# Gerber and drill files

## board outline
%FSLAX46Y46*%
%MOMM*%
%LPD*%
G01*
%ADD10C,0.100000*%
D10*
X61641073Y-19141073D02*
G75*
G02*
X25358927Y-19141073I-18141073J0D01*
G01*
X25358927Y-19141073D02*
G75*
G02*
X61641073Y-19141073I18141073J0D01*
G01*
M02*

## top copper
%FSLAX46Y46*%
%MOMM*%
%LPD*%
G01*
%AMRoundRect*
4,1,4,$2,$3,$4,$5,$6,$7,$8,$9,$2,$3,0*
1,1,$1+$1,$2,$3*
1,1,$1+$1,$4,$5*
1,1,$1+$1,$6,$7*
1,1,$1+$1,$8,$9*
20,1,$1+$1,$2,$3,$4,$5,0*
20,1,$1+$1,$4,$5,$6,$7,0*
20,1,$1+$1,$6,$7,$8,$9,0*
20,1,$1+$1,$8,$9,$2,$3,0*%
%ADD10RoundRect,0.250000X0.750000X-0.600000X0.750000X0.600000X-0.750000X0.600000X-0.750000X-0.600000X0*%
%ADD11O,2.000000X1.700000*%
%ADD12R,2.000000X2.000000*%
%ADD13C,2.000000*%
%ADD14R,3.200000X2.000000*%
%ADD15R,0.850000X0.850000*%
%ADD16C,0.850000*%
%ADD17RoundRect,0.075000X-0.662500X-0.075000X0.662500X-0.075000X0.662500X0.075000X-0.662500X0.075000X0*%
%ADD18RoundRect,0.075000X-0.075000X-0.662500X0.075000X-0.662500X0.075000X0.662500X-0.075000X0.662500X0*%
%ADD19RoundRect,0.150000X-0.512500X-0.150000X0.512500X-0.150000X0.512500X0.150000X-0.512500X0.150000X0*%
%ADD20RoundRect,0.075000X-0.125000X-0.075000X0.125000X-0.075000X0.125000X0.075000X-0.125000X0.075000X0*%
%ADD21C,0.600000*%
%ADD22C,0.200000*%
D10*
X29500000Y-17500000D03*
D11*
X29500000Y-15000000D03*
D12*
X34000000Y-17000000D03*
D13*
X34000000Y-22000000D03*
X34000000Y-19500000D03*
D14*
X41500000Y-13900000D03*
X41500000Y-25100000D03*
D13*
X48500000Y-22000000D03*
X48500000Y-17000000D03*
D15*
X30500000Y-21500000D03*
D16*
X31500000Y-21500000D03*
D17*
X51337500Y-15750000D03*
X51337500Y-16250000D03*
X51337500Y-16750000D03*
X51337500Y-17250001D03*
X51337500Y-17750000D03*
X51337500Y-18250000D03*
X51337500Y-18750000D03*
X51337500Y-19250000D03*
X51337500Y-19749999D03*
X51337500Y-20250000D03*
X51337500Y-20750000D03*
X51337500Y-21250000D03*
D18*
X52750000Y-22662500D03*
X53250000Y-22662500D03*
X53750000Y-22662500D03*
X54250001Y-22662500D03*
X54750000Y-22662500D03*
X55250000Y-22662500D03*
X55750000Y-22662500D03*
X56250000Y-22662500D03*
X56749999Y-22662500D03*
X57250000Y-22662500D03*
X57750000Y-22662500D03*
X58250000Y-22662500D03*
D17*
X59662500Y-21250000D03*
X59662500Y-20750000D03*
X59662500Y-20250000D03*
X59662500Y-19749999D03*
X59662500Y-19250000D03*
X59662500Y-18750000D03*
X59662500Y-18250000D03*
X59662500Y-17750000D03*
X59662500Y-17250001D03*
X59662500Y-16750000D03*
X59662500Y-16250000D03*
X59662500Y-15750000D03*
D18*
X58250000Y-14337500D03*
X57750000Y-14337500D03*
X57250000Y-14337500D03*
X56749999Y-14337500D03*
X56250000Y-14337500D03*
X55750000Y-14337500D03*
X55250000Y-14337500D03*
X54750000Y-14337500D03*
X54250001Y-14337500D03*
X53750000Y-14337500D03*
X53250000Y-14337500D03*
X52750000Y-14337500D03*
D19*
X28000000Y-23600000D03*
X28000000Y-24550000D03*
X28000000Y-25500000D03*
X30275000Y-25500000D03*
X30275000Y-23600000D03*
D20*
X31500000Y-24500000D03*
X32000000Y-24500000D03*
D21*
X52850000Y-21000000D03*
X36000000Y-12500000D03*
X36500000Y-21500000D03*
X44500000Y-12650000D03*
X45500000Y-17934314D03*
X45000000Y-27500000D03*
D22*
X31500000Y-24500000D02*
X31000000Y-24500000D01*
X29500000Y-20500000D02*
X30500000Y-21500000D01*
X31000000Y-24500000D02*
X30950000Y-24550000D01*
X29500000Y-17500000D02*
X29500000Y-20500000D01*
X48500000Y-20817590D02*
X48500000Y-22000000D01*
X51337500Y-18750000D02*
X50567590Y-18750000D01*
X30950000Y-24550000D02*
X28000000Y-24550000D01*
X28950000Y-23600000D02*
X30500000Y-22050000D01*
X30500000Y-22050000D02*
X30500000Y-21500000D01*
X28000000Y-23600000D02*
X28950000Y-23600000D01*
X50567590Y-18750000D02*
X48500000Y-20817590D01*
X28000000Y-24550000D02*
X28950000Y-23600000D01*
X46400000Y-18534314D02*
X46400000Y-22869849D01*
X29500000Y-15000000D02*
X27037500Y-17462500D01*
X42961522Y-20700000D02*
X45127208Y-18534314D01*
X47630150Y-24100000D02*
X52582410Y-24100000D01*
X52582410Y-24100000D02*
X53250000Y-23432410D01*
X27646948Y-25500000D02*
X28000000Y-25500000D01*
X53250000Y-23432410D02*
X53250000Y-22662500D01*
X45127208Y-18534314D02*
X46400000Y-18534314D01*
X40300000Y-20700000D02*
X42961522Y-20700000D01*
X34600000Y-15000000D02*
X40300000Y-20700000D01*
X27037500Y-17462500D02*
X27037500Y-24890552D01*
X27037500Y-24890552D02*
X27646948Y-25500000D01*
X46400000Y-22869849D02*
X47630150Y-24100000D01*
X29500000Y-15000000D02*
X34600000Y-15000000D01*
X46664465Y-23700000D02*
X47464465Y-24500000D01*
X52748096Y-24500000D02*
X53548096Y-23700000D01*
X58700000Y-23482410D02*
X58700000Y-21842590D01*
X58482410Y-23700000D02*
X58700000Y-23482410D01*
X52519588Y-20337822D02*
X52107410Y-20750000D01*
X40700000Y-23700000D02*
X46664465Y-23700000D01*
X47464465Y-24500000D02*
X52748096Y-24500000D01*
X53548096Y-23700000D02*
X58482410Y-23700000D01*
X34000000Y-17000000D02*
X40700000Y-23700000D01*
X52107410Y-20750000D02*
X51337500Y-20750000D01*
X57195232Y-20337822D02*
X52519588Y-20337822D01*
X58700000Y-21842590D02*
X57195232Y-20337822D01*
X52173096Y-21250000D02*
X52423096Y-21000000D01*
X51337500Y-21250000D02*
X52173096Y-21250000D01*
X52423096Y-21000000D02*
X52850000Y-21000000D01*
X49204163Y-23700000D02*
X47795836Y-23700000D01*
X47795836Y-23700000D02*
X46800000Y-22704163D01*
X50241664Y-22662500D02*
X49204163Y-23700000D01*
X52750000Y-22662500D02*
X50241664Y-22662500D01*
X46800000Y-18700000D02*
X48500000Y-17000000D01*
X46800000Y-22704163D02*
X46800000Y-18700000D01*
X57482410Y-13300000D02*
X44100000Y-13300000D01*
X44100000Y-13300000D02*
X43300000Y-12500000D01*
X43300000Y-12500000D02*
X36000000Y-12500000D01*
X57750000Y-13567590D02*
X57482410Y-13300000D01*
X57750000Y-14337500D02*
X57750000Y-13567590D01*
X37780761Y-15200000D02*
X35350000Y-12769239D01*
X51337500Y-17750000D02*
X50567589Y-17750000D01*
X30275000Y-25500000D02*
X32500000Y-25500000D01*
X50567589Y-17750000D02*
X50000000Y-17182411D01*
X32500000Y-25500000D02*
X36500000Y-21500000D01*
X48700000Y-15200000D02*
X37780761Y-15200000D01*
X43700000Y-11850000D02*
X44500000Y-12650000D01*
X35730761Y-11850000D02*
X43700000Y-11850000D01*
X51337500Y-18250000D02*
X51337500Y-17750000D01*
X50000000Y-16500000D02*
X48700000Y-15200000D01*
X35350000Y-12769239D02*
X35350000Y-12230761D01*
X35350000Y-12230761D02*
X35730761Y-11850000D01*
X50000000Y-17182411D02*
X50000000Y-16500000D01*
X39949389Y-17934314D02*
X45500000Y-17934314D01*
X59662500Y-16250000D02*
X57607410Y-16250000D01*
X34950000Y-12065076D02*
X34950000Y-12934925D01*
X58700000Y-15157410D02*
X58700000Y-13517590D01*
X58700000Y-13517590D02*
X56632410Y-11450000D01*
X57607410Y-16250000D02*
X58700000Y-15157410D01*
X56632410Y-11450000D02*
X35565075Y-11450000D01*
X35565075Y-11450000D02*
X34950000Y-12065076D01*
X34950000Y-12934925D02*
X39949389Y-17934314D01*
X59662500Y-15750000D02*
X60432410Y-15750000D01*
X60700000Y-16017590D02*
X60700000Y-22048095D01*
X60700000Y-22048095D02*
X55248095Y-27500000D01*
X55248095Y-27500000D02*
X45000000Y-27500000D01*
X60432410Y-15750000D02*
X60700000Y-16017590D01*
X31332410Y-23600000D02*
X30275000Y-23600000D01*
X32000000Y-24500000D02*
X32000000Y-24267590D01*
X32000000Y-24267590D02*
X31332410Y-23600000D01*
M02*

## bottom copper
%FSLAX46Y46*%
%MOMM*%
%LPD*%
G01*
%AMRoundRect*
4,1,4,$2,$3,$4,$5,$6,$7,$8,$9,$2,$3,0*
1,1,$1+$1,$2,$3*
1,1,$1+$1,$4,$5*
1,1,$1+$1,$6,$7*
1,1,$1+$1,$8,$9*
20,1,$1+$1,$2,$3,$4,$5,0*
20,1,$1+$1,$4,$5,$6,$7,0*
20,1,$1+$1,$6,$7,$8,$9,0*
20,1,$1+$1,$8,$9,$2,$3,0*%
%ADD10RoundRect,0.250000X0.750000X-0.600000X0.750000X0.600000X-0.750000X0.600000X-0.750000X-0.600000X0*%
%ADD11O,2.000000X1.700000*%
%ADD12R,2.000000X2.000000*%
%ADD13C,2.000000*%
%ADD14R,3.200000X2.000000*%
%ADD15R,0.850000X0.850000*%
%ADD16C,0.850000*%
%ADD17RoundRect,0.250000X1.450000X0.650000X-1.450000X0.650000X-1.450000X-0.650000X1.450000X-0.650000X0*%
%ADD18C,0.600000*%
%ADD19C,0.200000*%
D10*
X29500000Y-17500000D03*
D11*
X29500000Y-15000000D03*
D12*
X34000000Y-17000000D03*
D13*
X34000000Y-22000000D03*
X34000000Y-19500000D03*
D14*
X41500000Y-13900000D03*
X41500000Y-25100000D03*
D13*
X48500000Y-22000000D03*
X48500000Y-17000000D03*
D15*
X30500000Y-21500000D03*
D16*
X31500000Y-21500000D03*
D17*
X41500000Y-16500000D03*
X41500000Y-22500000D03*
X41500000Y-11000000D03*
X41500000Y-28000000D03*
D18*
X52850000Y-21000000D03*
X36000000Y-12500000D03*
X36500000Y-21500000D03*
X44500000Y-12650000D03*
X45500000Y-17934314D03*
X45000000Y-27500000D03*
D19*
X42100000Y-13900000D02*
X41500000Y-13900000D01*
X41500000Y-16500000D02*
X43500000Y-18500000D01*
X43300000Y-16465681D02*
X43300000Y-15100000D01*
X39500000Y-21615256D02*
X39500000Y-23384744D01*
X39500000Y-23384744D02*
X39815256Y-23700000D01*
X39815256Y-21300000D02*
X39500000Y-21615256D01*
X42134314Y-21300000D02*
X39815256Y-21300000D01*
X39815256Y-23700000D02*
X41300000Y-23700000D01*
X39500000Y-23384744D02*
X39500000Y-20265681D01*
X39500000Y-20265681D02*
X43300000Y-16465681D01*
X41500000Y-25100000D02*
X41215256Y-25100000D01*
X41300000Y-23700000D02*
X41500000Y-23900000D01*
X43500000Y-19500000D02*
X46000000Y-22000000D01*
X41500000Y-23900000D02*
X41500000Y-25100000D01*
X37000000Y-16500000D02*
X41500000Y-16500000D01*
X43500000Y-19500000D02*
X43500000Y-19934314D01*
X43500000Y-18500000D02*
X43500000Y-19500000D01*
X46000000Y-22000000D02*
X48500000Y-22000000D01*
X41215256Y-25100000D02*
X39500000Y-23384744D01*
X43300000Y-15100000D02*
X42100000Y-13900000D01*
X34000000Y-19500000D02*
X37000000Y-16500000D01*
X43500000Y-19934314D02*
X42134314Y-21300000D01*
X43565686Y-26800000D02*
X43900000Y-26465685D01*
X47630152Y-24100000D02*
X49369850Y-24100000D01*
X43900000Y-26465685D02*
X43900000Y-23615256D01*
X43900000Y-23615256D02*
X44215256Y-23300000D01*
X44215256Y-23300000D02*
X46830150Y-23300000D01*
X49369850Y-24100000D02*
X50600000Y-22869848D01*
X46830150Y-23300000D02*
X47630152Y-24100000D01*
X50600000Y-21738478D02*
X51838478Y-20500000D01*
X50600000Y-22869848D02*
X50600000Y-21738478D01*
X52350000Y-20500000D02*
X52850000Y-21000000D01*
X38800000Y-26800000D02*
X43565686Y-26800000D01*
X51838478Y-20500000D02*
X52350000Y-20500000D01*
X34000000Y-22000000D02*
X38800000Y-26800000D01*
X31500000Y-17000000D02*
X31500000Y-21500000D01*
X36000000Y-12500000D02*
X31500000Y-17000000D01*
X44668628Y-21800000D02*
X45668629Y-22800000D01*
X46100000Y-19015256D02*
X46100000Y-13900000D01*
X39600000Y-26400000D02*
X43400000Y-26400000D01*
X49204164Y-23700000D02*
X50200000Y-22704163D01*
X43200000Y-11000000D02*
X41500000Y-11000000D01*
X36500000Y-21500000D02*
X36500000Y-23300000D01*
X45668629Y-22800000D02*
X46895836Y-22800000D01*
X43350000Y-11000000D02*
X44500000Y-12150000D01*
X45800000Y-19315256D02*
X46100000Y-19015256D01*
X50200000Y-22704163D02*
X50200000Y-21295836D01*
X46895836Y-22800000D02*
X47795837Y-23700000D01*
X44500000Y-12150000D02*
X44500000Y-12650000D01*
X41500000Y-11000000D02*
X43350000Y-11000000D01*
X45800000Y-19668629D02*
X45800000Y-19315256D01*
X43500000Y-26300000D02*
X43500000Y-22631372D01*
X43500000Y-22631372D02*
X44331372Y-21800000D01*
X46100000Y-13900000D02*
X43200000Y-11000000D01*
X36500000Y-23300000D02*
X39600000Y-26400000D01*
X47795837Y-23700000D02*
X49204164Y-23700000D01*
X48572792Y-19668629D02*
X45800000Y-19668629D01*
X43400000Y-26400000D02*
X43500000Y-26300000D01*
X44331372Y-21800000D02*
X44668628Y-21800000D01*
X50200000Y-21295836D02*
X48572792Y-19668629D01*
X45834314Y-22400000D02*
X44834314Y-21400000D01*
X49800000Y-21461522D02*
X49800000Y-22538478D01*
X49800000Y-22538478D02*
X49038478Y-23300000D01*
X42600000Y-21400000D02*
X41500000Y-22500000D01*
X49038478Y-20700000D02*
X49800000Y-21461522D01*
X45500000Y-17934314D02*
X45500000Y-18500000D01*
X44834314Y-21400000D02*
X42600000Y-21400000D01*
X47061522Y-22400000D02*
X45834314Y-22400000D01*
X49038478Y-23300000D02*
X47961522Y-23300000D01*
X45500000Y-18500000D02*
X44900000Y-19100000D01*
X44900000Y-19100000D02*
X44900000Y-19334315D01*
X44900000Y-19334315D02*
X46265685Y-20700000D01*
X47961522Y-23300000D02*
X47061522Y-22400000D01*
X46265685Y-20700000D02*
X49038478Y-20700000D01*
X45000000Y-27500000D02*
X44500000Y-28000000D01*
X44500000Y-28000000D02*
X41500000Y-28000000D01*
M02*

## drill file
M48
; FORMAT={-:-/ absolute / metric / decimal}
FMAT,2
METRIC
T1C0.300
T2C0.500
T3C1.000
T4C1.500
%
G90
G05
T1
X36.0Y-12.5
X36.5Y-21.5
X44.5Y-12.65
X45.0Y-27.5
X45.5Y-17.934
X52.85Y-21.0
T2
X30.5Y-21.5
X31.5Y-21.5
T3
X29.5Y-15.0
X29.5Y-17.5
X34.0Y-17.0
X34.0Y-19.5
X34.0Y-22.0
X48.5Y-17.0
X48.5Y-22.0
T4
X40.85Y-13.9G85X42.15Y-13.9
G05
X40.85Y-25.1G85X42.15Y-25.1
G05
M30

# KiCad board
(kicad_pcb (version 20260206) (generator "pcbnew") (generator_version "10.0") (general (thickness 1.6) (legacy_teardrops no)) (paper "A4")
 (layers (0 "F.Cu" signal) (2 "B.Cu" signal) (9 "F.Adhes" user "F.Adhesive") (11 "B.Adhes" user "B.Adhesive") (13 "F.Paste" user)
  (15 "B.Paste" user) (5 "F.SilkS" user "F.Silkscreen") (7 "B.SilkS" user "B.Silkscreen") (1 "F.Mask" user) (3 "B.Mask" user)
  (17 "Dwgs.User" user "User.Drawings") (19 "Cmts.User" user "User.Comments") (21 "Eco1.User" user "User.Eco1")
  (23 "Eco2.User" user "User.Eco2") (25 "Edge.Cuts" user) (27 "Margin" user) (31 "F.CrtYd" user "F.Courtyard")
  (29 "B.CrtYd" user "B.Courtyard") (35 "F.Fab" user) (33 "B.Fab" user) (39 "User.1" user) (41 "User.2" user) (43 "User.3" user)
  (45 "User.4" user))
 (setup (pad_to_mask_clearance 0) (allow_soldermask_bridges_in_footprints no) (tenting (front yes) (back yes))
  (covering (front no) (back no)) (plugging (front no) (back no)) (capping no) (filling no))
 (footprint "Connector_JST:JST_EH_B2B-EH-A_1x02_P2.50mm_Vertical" (layer "F.Cu") (at 29.5 17.5 90)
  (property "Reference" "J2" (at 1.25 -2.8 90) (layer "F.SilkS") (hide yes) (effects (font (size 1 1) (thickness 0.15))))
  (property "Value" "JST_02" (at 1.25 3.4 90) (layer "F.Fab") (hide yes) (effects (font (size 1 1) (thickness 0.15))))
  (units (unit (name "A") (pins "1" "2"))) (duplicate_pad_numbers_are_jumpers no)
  (pad "1" thru_hole roundrect (at 0 0 90) (size 1.7 2) (drill 1) (layers "*.Cu" "*.Mask") (remove_unused_layers no)
   (roundrect_rratio 0.147059) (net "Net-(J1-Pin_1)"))
  (pad "2" thru_hole oval (at 2.5 0 90) (size 1.7 2) (drill 1) (layers "*.Cu" "*.Mask") (remove_unused_layers no) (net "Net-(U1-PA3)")))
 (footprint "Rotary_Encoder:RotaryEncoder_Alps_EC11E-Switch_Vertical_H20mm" (layer "F.Cu") (at 34 17)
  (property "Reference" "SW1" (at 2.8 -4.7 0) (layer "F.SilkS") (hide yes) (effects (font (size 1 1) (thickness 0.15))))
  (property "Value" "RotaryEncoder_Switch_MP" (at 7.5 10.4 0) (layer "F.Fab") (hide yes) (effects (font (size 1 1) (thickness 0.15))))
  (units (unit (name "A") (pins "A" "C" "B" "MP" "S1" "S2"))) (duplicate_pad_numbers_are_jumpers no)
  (pad "A" thru_hole rect (at 0 0) (size 2 2) (drill 1) (layers "*.Cu" "*.Mask") (remove_unused_layers no) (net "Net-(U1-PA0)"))
  (pad "B" thru_hole circle (at 0 5) (size 2 2) (drill 1) (layers "*.Cu" "*.Mask") (remove_unused_layers no) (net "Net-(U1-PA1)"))
  (pad "C" thru_hole circle (at 0 2.5) (size 2 2) (drill 1) (layers "*.Cu" "*.Mask") (remove_unused_layers no) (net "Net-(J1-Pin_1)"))
  (pad "MP" thru_hole rect (at 7.5 -3.1) (size 3.2 2) (drill oval 2.8 1.5) (layers "*.Cu" "*.Mask") (remove_unused_layers no)
   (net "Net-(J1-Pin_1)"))
  (pad "MP" thru_hole rect (at 7.5 8.1) (size 3.2 2) (drill oval 2.8 1.5) (layers "*.Cu" "*.Mask") (remove_unused_layers no)
   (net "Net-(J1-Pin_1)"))
  (pad "S1" thru_hole circle (at 14.5 5) (size 2 2) (drill 1) (layers "*.Cu" "*.Mask") (remove_unused_layers no) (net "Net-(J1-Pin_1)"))
  (pad "S2" thru_hole circle (at 14.5 0) (size 2 2) (drill 1) (layers "*.Cu" "*.Mask") (remove_unused_layers no) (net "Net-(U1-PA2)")))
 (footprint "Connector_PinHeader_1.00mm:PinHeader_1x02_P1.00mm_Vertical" (layer "F.Cu") (at 30.5 21.5 90)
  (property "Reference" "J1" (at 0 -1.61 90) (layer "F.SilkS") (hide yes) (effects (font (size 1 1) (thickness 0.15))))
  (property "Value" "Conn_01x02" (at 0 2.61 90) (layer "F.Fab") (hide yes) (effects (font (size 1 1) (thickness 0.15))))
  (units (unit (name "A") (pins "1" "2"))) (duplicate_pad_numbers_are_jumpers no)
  (pad "1" thru_hole rect (at 0 0 90) (size 0.85 0.85) (drill 0.5) (layers "*.Cu" "*.Mask") (remove_unused_layers no) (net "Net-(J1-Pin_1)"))
  (pad "2" thru_hole circle (at 0 1 90) (size 0.85 0.85) (drill 0.5) (layers "*.Cu" "*.Mask") (remove_unused_layers no)
   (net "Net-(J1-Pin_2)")))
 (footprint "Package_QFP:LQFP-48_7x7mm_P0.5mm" (layer "F.Cu") (at 55.5 18.5)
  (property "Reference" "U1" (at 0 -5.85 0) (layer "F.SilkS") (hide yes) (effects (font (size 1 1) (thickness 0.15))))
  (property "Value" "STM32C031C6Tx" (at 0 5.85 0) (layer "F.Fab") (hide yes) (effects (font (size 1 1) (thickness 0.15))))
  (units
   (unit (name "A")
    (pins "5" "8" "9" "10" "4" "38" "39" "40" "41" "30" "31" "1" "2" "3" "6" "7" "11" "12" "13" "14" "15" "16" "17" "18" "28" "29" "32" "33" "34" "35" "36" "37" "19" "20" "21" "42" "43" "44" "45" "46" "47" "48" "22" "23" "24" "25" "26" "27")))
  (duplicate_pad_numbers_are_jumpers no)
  (pad "1" smd roundrect (at -4.1625 -2.75) (size 1.475 0.3) (layers "F.Cu" "F.Mask" "F.Paste") (roundrect_rratio 0.25)
   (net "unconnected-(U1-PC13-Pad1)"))
  (pad "2" smd roundrect (at -4.1625 -2.25) (size 1.475 0.3) (layers "F.Cu" "F.Mask" "F.Paste") (roundrect_rratio 0.25)
   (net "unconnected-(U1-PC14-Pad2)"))
  (pad "3" smd roundrect (at -4.1625 -1.75) (size 1.475 0.3) (layers "F.Cu" "F.Mask" "F.Paste") (roundrect_rratio 0.25)
   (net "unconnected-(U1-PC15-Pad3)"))
  (pad "4" smd roundrect (at -4.1625 -1.249999) (size 1.475 0.3) (layers "F.Cu" "F.Mask" "F.Paste") (roundrect_rratio 0.25)
   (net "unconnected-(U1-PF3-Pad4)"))
  (pad "5" smd roundrect (at -4.1625 -0.75) (size 1.475 0.3) (layers "F.Cu" "F.Mask" "F.Paste") (roundrect_rratio 0.25) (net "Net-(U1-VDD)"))
  (pad "6" smd roundrect (at -4.1625 -0.25) (size 1.475 0.3) (layers "F.Cu" "F.Mask" "F.Paste") (roundrect_rratio 0.25) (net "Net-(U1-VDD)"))
  (pad "7" smd roundrect (at -4.1625 0.25) (size 1.475 0.3) (layers "F.Cu" "F.Mask" "F.Paste") (roundrect_rratio 0.25)
   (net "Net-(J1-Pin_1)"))
  (pad "8" smd roundrect (at -4.1625 0.75) (size 1.475 0.3) (layers "F.Cu" "F.Mask" "F.Paste") (roundrect_rratio 0.25)
   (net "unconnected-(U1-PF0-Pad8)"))
  (pad "9" smd roundrect (at -4.1625 1.249999) (size 1.475 0.3) (layers "F.Cu" "F.Mask" "F.Paste") (roundrect_rratio 0.25)
   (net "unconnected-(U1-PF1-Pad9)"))
  (pad "10" smd roundrect (at -4.1625 1.75) (size 1.475 0.3) (layers "F.Cu" "F.Mask" "F.Paste") (roundrect_rratio 0.25)
   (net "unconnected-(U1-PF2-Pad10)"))
  (pad "11" smd roundrect (at -4.1625 2.25) (size 1.475 0.3) (layers "F.Cu" "F.Mask" "F.Paste") (roundrect_rratio 0.25) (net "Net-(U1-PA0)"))
  (pad "12" smd roundrect (at -4.1625 2.75) (size 1.475 0.3) (layers "F.Cu" "F.Mask" "F.Paste") (roundrect_rratio 0.25) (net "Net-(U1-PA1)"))
  (pad "13" smd roundrect (at -2.75 4.1625) (size 0.3 1.475) (layers "F.Cu" "F.Mask" "F.Paste") (roundrect_rratio 0.25) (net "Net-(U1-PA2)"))
  (pad "14" smd roundrect (at -2.25 4.1625) (size 0.3 1.475) (layers "F.Cu" "F.Mask" "F.Paste") (roundrect_rratio 0.25) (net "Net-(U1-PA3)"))
  (pad "15" smd roundrect (at -1.75 4.1625) (size 0.3 1.475) (layers "F.Cu" "F.Mask" "F.Paste") (roundrect_rratio 0.25)
   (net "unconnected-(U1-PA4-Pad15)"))
  (pad "16" smd roundrect (at -1.249999 4.1625) (size 0.3 1.475) (layers "F.Cu" "F.Mask" "F.Paste") (roundrect_rratio 0.25)
   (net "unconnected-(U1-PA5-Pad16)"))
  (pad "17" smd roundrect (at -0.75 4.1625) (size 0.3 1.475) (layers "F.Cu" "F.Mask" "F.Paste") (roundrect_rratio 0.25)
   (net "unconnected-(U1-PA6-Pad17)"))
  (pad "18" smd roundrect (at -0.25 4.1625) (size 0.3 1.475) (layers "F.Cu" "F.Mask" "F.Paste") (roundrect_rratio 0.25)
   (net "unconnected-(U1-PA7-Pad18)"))
  (pad "19" smd roundrect (at 0.25 4.1625) (size 0.3 1.475) (layers "F.Cu" "F.Mask" "F.Paste") (roundrect_rratio 0.25)
   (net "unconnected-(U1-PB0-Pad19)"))
  (pad "20" smd roundrect (at 0.75 4.1625) (size 0.3 1.475) (layers "F.Cu" "F.Mask" "F.Paste") (roundrect_rratio 0.25)
   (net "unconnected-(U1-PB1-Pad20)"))
  (pad "21" smd roundrect (at 1.249999 4.1625) (size 0.3 1.475) (layers "F.Cu" "F.Mask" "F.Paste") (roundrect_rratio 0.25)
   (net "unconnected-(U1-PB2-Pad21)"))
  (pad "22" smd roundrect (at 1.75 4.1625) (size 0.3 1.475) (layers "F.Cu" "F.Mask" "F.Paste") (roundrect_rratio 0.25)
   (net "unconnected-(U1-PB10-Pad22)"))
  (pad "23" smd roundrect (at 2.25 4.1625) (size 0.3 1.475) (layers "F.Cu" "F.Mask" "F.Paste") (roundrect_rratio 0.25)
   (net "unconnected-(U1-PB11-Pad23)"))
  (pad "24" smd roundrect (at 2.75 4.1625) (size 0.3 1.475) (layers "F.Cu" "F.Mask" "F.Paste") (roundrect_rratio 0.25)
   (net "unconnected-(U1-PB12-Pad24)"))
  (pad "25" smd roundrect (at 4.1625 2.75) (size 1.475 0.3) (layers "F.Cu" "F.Mask" "F.Paste") (roundrect_rratio 0.25)
   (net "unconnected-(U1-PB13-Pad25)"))
  (pad "26" smd roundrect (at 4.1625 2.25) (size 1.475 0.3) (layers "F.Cu" "F.Mask" "F.Paste") (roundrect_rratio 0.25)
   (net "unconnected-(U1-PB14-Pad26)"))
  (pad "27" smd roundrect (at 4.1625 1.75) (size 1.475 0.3) (layers "F.Cu" "F.Mask" "F.Paste") (roundrect_rratio 0.25)
   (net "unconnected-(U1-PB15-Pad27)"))
  (pad "28" smd roundrect (at 4.1625 1.249999) (size 1.475 0.3) (layers "F.Cu" "F.Mask" "F.Paste") (roundrect_rratio 0.25)
   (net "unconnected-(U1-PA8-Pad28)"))
  (pad "29" smd roundrect (at 4.1625 0.75) (size 1.475 0.3) (layers "F.Cu" "F.Mask" "F.Paste") (roundrect_rratio 0.25)
   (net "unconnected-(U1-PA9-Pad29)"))
  (pad "30" smd roundrect (at 4.1625 0.25) (size 1.475 0.3) (layers "F.Cu" "F.Mask" "F.Paste") (roundrect_rratio 0.25)
   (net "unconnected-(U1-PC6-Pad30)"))
  (pad "31" smd roundrect (at 4.1625 -0.25) (size 1.475 0.3) (layers "F.Cu" "F.Mask" "F.Paste") (roundrect_rratio 0.25)
   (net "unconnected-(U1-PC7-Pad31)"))
  (pad "32" smd roundrect (at 4.1625 -0.75) (size 1.475 0.3) (layers "F.Cu" "F.Mask" "F.Paste") (roundrect_rratio 0.25)
   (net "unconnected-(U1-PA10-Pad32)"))
  (pad "33" smd roundrect (at 4.1625 -1.249999) (size 1.475 0.3) (layers "F.Cu" "F.Mask" "F.Paste") (roundrect_rratio 0.25)
   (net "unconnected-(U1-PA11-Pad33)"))
  (pad "34" smd roundrect (at 4.1625 -1.75) (size 1.475 0.3) (layers "F.Cu" "F.Mask" "F.Paste") (roundrect_rratio 0.25)
   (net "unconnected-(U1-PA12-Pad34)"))
  (pad "35" smd roundrect (at 4.1625 -2.25) (size 1.475 0.3) (layers "F.Cu" "F.Mask" "F.Paste") (roundrect_rratio 0.25)
   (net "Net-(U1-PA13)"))
  (pad "36" smd roundrect (at 4.1625 -2.75) (size 1.475 0.3) (layers "F.Cu" "F.Mask" "F.Paste") (roundrect_rratio 0.25)
   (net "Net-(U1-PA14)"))
  (pad "37" smd roundrect (at 2.75 -4.1625) (size 0.3 1.475) (layers "F.Cu" "F.Mask" "F.Paste") (roundrect_rratio 0.25)
   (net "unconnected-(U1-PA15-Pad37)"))
  (pad "38" smd roundrect (at 2.25 -4.1625) (size 0.3 1.475) (layers "F.Cu" "F.Mask" "F.Paste") (roundrect_rratio 0.25)
   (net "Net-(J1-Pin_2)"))
  (pad "39" smd roundrect (at 1.75 -4.1625) (size 0.3 1.475) (layers "F.Cu" "F.Mask" "F.Paste") (roundrect_rratio 0.25)
   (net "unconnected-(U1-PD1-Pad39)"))
  (pad "40" smd roundrect (at 1.249999 -4.1625) (size 0.3 1.475) (layers "F.Cu" "F.Mask" "F.Paste") (roundrect_rratio 0.25)
   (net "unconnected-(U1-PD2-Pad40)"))
  (pad "41" smd roundrect (at 0.75 -4.1625) (size 0.3 1.475) (layers "F.Cu" "F.Mask" "F.Paste") (roundrect_rratio 0.25)
   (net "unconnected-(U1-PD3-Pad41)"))
  (pad "42" smd roundrect (at 0.25 -4.1625) (size 0.3 1.475) (layers "F.Cu" "F.Mask" "F.Paste") (roundrect_rratio 0.25)
   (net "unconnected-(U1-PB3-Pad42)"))
  (pad "43" smd roundrect (at -0.25 -4.1625) (size 0.3 1.475) (layers "F.Cu" "F.Mask" "F.Paste") (roundrect_rratio 0.25)
   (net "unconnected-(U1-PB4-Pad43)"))
  (pad "44" smd roundrect (at -0.75 -4.1625) (size 0.3 1.475) (layers "F.Cu" "F.Mask" "F.Paste") (roundrect_rratio 0.25)
   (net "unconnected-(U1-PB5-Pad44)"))
  (pad "45" smd roundrect (at -1.249999 -4.1625) (size 0.3 1.475) (layers "F.Cu" "F.Mask" "F.Paste") (roundrect_rratio 0.25)
   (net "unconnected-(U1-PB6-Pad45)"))
  (pad "46" smd roundrect (at -1.75 -4.1625) (size 0.3 1.475) (layers "F.Cu" "F.Mask" "F.Paste") (roundrect_rratio 0.25)
   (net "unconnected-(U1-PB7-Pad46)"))
  (pad "47" smd roundrect (at -2.25 -4.1625) (size 0.3 1.475) (layers "F.Cu" "F.Mask" "F.Paste") (roundrect_rratio 0.25)
   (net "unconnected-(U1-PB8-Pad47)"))
  (pad "48" smd roundrect (at -2.75 -4.1625) (size 0.3 1.475) (layers "F.Cu" "F.Mask" "F.Paste") (roundrect_rratio 0.25)
   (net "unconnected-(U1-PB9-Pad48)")))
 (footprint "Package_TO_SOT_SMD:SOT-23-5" (layer "F.Cu") (at 29.1375 24.55)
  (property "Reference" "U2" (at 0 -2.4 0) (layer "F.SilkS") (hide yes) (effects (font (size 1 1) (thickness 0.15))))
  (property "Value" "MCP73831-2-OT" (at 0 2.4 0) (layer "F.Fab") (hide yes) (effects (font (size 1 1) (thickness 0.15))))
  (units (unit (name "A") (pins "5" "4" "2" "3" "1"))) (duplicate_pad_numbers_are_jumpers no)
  (pad "1" smd roundrect (at -1.1375 -0.95) (size 1.325 0.6) (layers "F.Cu" "F.Mask" "F.Paste") (roundrect_rratio 0.25)
   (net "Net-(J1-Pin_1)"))
  (pad "2" smd roundrect (at -1.1375 0) (size 1.325 0.6) (layers "F.Cu" "F.Mask" "F.Paste") (roundrect_rratio 0.25) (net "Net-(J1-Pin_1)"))
  (pad "3" smd roundrect (at -1.1375 0.95) (size 1.325 0.6) (layers "F.Cu" "F.Mask" "F.Paste") (roundrect_rratio 0.25) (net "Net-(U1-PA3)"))
  (pad "4" smd roundrect (at 1.1375 0.95) (size 1.325 0.6) (layers "F.Cu" "F.Mask" "F.Paste") (roundrect_rratio 0.25) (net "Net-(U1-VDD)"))
  (pad "5" smd roundrect (at 1.1375 -0.95) (size 1.325 0.6) (layers "F.Cu" "F.Mask" "F.Paste") (roundrect_rratio 0.25) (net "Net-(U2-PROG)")))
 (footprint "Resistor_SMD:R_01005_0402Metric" (layer "F.Cu") (at 31.75 24.5)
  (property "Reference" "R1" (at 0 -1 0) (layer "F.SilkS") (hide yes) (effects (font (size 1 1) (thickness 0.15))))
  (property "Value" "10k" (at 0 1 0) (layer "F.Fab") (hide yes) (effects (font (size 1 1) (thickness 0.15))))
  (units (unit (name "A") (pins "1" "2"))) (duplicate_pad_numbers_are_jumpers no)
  (pad "" smd roundrect (at -0.275 0) (size 0.27 0.27) (layers "F.Paste") (roundrect_rratio 0.25))
  (pad "" smd roundrect (at 0.275 0) (size 0.27 0.27) (layers "F.Paste") (roundrect_rratio 0.25))
  (pad "1" smd roundrect (at -0.25 0) (size 0.4 0.3) (layers "F.Cu" "F.Mask") (roundrect_rratio 0.25) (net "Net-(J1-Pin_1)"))
  (pad "2" smd roundrect (at 0.25 0) (size 0.4 0.3) (layers "F.Cu" "F.Mask") (roundrect_rratio 0.25) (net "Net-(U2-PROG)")))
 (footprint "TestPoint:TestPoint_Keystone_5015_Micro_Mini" (layer "B.Cu") (at 41.5 16.5 180)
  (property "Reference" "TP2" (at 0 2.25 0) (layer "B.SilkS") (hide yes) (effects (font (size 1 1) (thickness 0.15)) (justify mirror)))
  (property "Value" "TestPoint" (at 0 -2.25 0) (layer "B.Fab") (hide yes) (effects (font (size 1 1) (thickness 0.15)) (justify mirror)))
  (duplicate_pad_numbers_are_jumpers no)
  (pad "1" smd roundrect (at 0 0 180) (size 3.4 1.8) (layers "B.Cu" "B.Mask" "B.Paste") (roundrect_rratio 0.1388888889)
   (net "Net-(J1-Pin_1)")))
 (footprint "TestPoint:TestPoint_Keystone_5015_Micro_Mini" (layer "B.Cu") (at 41.5 22.5 180)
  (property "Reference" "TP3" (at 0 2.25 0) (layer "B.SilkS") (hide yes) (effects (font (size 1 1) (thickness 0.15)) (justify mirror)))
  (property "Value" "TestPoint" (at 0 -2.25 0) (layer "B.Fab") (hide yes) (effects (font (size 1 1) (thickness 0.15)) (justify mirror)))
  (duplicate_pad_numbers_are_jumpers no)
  (pad "1" smd roundrect (at 0 0 180) (size 3.4 1.8) (layers "B.Cu" "B.Mask" "B.Paste") (roundrect_rratio 0.1388888889)
   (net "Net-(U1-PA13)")))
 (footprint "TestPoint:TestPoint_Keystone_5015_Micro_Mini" (layer "B.Cu") (at 41.5 11 180)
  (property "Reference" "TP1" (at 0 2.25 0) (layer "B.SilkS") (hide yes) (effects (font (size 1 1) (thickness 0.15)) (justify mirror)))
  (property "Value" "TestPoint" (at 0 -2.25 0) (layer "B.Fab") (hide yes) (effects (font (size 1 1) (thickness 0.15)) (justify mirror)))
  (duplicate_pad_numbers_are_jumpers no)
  (pad "1" smd roundrect (at 0 0 180) (size 3.4 1.8) (layers "B.Cu" "B.Mask" "B.Paste") (roundrect_rratio 0.1388888889) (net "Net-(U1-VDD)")))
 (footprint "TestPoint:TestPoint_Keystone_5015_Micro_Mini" (layer "B.Cu") (at 41.5 28 180)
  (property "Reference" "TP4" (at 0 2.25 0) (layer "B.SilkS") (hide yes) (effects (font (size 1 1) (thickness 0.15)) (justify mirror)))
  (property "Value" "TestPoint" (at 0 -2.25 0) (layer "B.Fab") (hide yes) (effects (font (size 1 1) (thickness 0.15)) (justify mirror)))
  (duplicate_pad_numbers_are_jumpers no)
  (pad "1" smd roundrect (at 0 0 180) (size 3.4 1.8) (layers "B.Cu" "B.Mask" "B.Paste") (roundrect_rratio 0.1388888889)
   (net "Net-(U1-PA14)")))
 (gr_circle (center 43.5 19.141073) (end 54.5 4.715453) (stroke (width 0.1) (type default)) (fill no) (layer "Edge.Cuts"))
 (segment (start 31.5 24.5) (end 31 24.5) (width 0.2) (layer "F.Cu") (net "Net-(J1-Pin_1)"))
 (segment (start 29.5 20.5) (end 30.5 21.5) (width 0.2) (layer "F.Cu") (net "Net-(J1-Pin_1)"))
 (segment (start 31 24.5) (end 30.95 24.55) (width 0.2) (layer "F.Cu") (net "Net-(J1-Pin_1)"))
 (segment (start 29.5 17.5) (end 29.5 20.5) (width 0.2) (layer "F.Cu") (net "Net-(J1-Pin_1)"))
 (segment (start 48.5 20.81759) (end 48.5 22) (width 0.2) (layer "F.Cu") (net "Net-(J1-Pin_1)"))
 (segment (start 51.3375 18.75) (end 50.56759 18.75) (width 0.2) (layer "F.Cu") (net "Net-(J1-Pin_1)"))
 (segment (start 30.95 24.55) (end 28 24.55) (width 0.2) (layer "F.Cu") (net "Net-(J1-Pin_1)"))
 (segment (start 28.95 23.6) (end 30.5 22.05) (width 0.2) (layer "F.Cu") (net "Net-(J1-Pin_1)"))
 (segment (start 30.5 22.05) (end 30.5 21.5) (width 0.2) (layer "F.Cu") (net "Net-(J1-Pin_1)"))
 (segment (start 28 23.6) (end 28.95 23.6) (width 0.2) (layer "F.Cu") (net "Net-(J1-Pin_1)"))
 (segment (start 50.56759 18.75) (end 48.5 20.81759) (width 0.2) (layer "F.Cu") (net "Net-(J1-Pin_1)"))
 (segment (start 28 24.55) (end 28.95 23.6) (width 0.2) (layer "F.Cu") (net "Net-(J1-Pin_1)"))
 (segment (start 42.1 13.9) (end 41.5 13.9) (width 0.2) (layer "B.Cu") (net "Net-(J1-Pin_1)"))
 (segment (start 41.5 16.5) (end 43.5 18.5) (width 0.2) (layer "B.Cu") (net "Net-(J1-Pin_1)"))
 (segment (start 43.3 16.465681) (end 43.3 15.1) (width 0.2) (layer "B.Cu") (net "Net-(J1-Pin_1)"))
 (segment (start 39.5 21.615256) (end 39.5 23.384744) (width 0.2) (layer "B.Cu") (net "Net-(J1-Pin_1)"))
 (segment (start 39.5 23.384744) (end 39.815256 23.7) (width 0.2) (layer "B.Cu") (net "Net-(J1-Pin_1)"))
 (segment (start 39.815256 21.3) (end 39.5 21.615256) (width 0.2) (layer "B.Cu") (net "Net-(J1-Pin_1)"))
 (segment (start 42.134314 21.3) (end 39.815256 21.3) (width 0.2) (layer "B.Cu") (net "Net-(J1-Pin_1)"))
 (segment (start 39.815256 23.7) (end 41.3 23.7) (width 0.2) (layer "B.Cu") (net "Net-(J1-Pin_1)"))
 (segment (start 39.5 23.384744) (end 39.5 20.265681) (width 0.2) (layer "B.Cu") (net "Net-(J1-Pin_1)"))
 (segment (start 39.5 20.265681) (end 43.3 16.465681) (width 0.2) (layer "B.Cu") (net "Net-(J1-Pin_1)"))
 (segment (start 41.5 25.1) (end 41.215256 25.1) (width 0.2) (layer "B.Cu") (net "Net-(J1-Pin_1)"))
 (segment (start 41.3 23.7) (end 41.5 23.9) (width 0.2) (layer "B.Cu") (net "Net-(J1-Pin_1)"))
 (segment (start 43.5 19.5) (end 46 22) (width 0.2) (layer "B.Cu") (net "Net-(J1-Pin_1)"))
 (segment (start 41.5 23.9) (end 41.5 25.1) (width 0.2) (layer "B.Cu") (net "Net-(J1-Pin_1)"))
 (segment (start 37 16.5) (end 41.5 16.5) (width 0.2) (layer "B.Cu") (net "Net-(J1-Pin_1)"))
 (segment (start 43.5 19.5) (end 43.5 19.934314) (width 0.2) (layer "B.Cu") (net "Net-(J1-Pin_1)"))
 (segment (start 43.5 18.5) (end 43.5 19.5) (width 0.2) (layer "B.Cu") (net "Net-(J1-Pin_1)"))
 (segment (start 46 22) (end 48.5 22) (width 0.2) (layer "B.Cu") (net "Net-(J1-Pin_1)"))
 (segment (start 41.215256 25.1) (end 39.5 23.384744) (width 0.2) (layer "B.Cu") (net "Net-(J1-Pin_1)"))
 (segment (start 43.3 15.1) (end 42.1 13.9) (width 0.2) (layer "B.Cu") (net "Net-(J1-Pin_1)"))
 (segment (start 34 19.5) (end 37 16.5) (width 0.2) (layer "B.Cu") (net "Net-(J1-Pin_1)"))
 (segment (start 43.5 19.934314) (end 42.134314 21.3) (width 0.2) (layer "B.Cu") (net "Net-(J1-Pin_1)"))
 (segment (start 46.4 18.534314) (end 46.4 22.869849) (width 0.2) (layer "F.Cu") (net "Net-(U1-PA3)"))
 (segment (start 29.5 15) (end 27.0375 17.4625) (width 0.2) (layer "F.Cu") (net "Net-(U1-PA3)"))
 (segment (start 42.961522 20.7) (end 45.127208 18.534314) (width 0.2) (layer "F.Cu") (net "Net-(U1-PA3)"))
 (segment (start 47.63015 24.1) (end 52.58241 24.1) (width 0.2) (layer "F.Cu") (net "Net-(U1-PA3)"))
 (segment (start 52.58241 24.1) (end 53.25 23.43241) (width 0.2) (layer "F.Cu") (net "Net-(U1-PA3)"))
 (segment (start 27.646948 25.5) (end 28 25.5) (width 0.2) (layer "F.Cu") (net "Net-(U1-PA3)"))
 (segment (start 53.25 23.43241) (end 53.25 22.6625) (width 0.2) (layer "F.Cu") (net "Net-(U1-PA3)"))
 (segment (start 45.127208 18.534314) (end 46.4 18.534314) (width 0.2) (layer "F.Cu") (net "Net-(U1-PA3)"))
 (segment (start 40.3 20.7) (end 42.961522 20.7) (width 0.2) (layer "F.Cu") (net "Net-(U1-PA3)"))
 (segment (start 34.6 15) (end 40.3 20.7) (width 0.2) (layer "F.Cu") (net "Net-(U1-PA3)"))
 (segment (start 27.0375 17.4625) (end 27.0375 24.890552) (width 0.2) (layer "F.Cu") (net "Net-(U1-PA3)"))
 (segment (start 27.0375 24.890552) (end 27.646948 25.5) (width 0.2) (layer "F.Cu") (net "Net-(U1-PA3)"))
 (segment (start 46.4 22.869849) (end 47.63015 24.1) (width 0.2) (layer "F.Cu") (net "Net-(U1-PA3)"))
 (segment (start 29.5 15) (end 34.6 15) (width 0.2) (layer "F.Cu") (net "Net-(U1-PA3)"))
 (segment (start 46.664465 23.7) (end 47.464465 24.5) (width 0.2) (layer "F.Cu") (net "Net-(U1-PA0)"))
 (segment (start 52.748096 24.5) (end 53.548096 23.7) (width 0.2) (layer "F.Cu") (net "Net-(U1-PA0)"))
 (segment (start 58.7 23.48241) (end 58.7 21.84259) (width 0.2) (layer "F.Cu") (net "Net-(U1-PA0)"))
 (segment (start 58.48241 23.7) (end 58.7 23.48241) (width 0.2) (layer "F.Cu") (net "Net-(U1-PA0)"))
 (segment (start 52.519588 20.337822) (end 52.10741 20.75) (width 0.2) (layer "F.Cu") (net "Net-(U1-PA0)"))
 (segment (start 40.7 23.7) (end 46.664465 23.7) (width 0.2) (layer "F.Cu") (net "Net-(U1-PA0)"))
 (segment (start 47.464465 24.5) (end 52.748096 24.5) (width 0.2) (layer "F.Cu") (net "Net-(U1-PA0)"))
 (segment (start 53.548096 23.7) (end 58.48241 23.7) (width 0.2) (layer "F.Cu") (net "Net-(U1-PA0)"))
 (segment (start 34 17) (end 40.7 23.7) (width 0.2) (layer "F.Cu") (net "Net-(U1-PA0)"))
 (segment (start 52.10741 20.75) (end 51.3375 20.75) (width 0.2) (layer "F.Cu") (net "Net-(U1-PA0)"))
 (segment (start 57.195232 20.337822) (end 52.519588 20.337822) (width 0.2) (layer "F.Cu") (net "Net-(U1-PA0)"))
 (segment (start 58.7 21.84259) (end 57.195232 20.337822) (width 0.2) (layer "F.Cu") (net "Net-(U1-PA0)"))
 (segment (start 52.173096 21.25) (end 52.423096 21) (width 0.2) (layer "F.Cu") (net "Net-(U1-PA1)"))
 (segment (start 51.3375 21.25) (end 52.173096 21.25) (width 0.2) (layer "F.Cu") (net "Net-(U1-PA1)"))
 (segment (start 52.423096 21) (end 52.85 21) (width 0.2) (layer "F.Cu") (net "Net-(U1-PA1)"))
 (via (at 52.85 21) (size 0.6) (drill 0.3) (layers "F.Cu" "B.Cu") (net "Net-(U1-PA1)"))
 (segment (start 43.565686 26.8) (end 43.9 26.465685) (width 0.2) (layer "B.Cu") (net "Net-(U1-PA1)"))
 (segment (start 47.630152 24.1) (end 49.36985 24.1) (width 0.2) (layer "B.Cu") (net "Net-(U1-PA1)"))
 (segment (start 43.9 26.465685) (end 43.9 23.615256) (width 0.2) (layer "B.Cu") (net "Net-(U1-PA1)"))
 (segment (start 43.9 23.615256) (end 44.215256 23.3) (width 0.2) (layer "B.Cu") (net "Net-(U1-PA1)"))
 (segment (start 44.215256 23.3) (end 46.83015 23.3) (width 0.2) (layer "B.Cu") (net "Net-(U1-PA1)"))
 (segment (start 49.36985 24.1) (end 50.6 22.869848) (width 0.2) (layer "B.Cu") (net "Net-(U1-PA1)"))
 (segment (start 46.83015 23.3) (end 47.630152 24.1) (width 0.2) (layer "B.Cu") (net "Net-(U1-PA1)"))
 (segment (start 50.6 21.738478) (end 51.838478 20.5) (width 0.2) (layer "B.Cu") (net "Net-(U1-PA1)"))
 (segment (start 50.6 22.869848) (end 50.6 21.738478) (width 0.2) (layer "B.Cu") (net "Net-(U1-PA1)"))
 (segment (start 52.35 20.5) (end 52.85 21) (width 0.2) (layer "B.Cu") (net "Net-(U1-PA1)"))
 (segment (start 38.8 26.8) (end 43.565686 26.8) (width 0.2) (layer "B.Cu") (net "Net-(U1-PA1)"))
 (segment (start 51.838478 20.5) (end 52.35 20.5) (width 0.2) (layer "B.Cu") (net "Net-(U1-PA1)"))
 (segment (start 34 22) (end 38.8 26.8) (width 0.2) (layer "B.Cu") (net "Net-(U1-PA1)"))
 (segment (start 49.204163 23.7) (end 47.795836 23.7) (width 0.2) (layer "F.Cu") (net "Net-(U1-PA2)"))
 (segment (start 47.795836 23.7) (end 46.8 22.704163) (width 0.2) (layer "F.Cu") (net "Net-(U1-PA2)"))
 (segment (start 50.241664 22.6625) (end 49.204163 23.7) (width 0.2) (layer "F.Cu") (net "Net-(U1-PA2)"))
 (segment (start 52.75 22.6625) (end 50.241664 22.6625) (width 0.2) (layer "F.Cu") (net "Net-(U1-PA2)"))
 (segment (start 46.8 18.7) (end 48.5 17) (width 0.2) (layer "F.Cu") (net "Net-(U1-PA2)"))
 (segment (start 46.8 22.704163) (end 46.8 18.7) (width 0.2) (layer "F.Cu") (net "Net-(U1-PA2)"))
 (segment (start 57.48241 13.3) (end 44.1 13.3) (width 0.2) (layer "F.Cu") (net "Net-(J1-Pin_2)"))
 (segment (start 44.1 13.3) (end 43.3 12.5) (width 0.2) (layer "F.Cu") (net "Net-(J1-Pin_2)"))
 (segment (start 43.3 12.5) (end 36 12.5) (width 0.2) (layer "F.Cu") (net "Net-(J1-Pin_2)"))
 (segment (start 57.75 13.56759) (end 57.48241 13.3) (width 0.2) (layer "F.Cu") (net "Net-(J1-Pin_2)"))
 (segment (start 57.75 14.3375) (end 57.75 13.56759) (width 0.2) (layer "F.Cu") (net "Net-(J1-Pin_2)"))
 (via (at 36 12.5) (size 0.6) (drill 0.3) (layers "F.Cu" "B.Cu") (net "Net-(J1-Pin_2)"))
 (segment (start 31.5 17) (end 31.5 21.5) (width 0.2) (layer "B.Cu") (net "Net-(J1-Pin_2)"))
 (segment (start 36 12.5) (end 31.5 17) (width 0.2) (layer "B.Cu") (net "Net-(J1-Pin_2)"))
 (segment (start 37.780761 15.2) (end 35.35 12.769239) (width 0.2) (layer "F.Cu") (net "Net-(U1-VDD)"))
 (segment (start 51.3375 17.75) (end 50.567589 17.75) (width 0.2) (layer "F.Cu") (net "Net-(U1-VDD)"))
 (segment (start 30.275 25.5) (end 32.5 25.5) (width 0.2) (layer "F.Cu") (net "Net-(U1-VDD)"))
 (segment (start 50.567589 17.75) (end 50 17.182411) (width 0.2) (layer "F.Cu") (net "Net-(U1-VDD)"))
 (segment (start 32.5 25.5) (end 36.5 21.5) (width 0.2) (layer "F.Cu") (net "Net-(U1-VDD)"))
 (segment (start 48.7 15.2) (end 37.780761 15.2) (width 0.2) (layer "F.Cu") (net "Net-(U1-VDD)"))
 (segment (start 43.7 11.85) (end 44.5 12.65) (width 0.2) (layer "F.Cu") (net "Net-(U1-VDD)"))
 (segment (start 35.730761 11.85) (end 43.7 11.85) (width 0.2) (layer "F.Cu") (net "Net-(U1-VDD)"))
 (segment (start 51.3375 18.25) (end 51.3375 17.75) (width 0.2) (layer "F.Cu") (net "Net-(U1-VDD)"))
 (segment (start 50 16.5) (end 48.7 15.2) (width 0.2) (layer "F.Cu") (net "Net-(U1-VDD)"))
 (segment (start 35.35 12.769239) (end 35.35 12.230761) (width 0.2) (layer "F.Cu") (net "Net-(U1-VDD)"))
 (segment (start 35.35 12.230761) (end 35.730761 11.85) (width 0.2) (layer "F.Cu") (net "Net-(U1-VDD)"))
 (segment (start 50 17.182411) (end 50 16.5) (width 0.2) (layer "F.Cu") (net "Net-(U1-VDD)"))
 (via (at 36.5 21.5) (size 0.6) (drill 0.3) (layers "F.Cu" "B.Cu") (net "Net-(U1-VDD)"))
 (via (at 44.5 12.65) (size 0.6) (drill 0.3) (layers "F.Cu" "B.Cu") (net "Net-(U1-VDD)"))
 (segment (start 44.668628 21.8) (end 45.668629 22.8) (width 0.2) (layer "B.Cu") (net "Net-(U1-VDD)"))
 (segment (start 46.1 19.015256) (end 46.1 13.9) (width 0.2) (layer "B.Cu") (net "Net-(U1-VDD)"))
 (segment (start 39.6 26.4) (end 43.4 26.4) (width 0.2) (layer "B.Cu") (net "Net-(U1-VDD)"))
 (segment (start 49.204164 23.7) (end 50.2 22.704163) (width 0.2) (layer "B.Cu") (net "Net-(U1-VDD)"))
 (segment (start 43.2 11) (end 41.5 11) (width 0.2) (layer "B.Cu") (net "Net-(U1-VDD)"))
 (segment (start 36.5 21.5) (end 36.5 23.3) (width 0.2) (layer "B.Cu") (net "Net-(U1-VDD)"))
 (segment (start 45.668629 22.8) (end 46.895836 22.8) (width 0.2) (layer "B.Cu") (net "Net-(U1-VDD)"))
 (segment (start 43.35 11) (end 44.5 12.15) (width 0.2) (layer "B.Cu") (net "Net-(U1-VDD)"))
 (segment (start 45.8 19.315256) (end 46.1 19.015256) (width 0.2) (layer "B.Cu") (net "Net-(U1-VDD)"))
 (segment (start 50.2 22.704163) (end 50.2 21.295836) (width 0.2) (layer "B.Cu") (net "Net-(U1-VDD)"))
 (segment (start 46.895836 22.8) (end 47.795837 23.7) (width 0.2) (layer "B.Cu") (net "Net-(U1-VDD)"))
 (segment (start 44.5 12.15) (end 44.5 12.65) (width 0.2) (layer "B.Cu") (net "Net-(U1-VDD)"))
 (segment (start 41.5 11) (end 43.35 11) (width 0.2) (layer "B.Cu") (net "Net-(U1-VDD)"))
 (segment (start 45.8 19.668629) (end 45.8 19.315256) (width 0.2) (layer "B.Cu") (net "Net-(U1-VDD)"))
 (segment (start 43.5 26.3) (end 43.5 22.631372) (width 0.2) (layer "B.Cu") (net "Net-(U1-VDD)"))
 (segment (start 43.5 22.631372) (end 44.331372 21.8) (width 0.2) (layer "B.Cu") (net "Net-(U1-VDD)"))
 (segment (start 46.1 13.9) (end 43.2 11) (width 0.2) (layer "B.Cu") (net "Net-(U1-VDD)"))
 (segment (start 36.5 23.3) (end 39.6 26.4) (width 0.2) (layer "B.Cu") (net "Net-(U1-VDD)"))
 (segment (start 47.795837 23.7) (end 49.204164 23.7) (width 0.2) (layer "B.Cu") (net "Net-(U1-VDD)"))
 (segment (start 48.572792 19.668629) (end 45.8 19.668629) (width 0.2) (layer "B.Cu") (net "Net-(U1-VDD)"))
 (segment (start 43.4 26.4) (end 43.5 26.3) (width 0.2) (layer "B.Cu") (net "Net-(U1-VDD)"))
 (segment (start 44.331372 21.8) (end 44.668628 21.8) (width 0.2) (layer "B.Cu") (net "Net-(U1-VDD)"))
 (segment (start 50.2 21.295836) (end 48.572792 19.668629) (width 0.2) (layer "B.Cu") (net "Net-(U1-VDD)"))
 (segment (start 39.949389 17.934314) (end 45.5 17.934314) (width 0.2) (layer "F.Cu") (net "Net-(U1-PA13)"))
 (segment (start 59.6625 16.25) (end 57.60741 16.25) (width 0.2) (layer "F.Cu") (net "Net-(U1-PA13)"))
 (segment (start 34.95 12.065076) (end 34.95 12.934925) (width 0.2) (layer "F.Cu") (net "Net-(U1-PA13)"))
 (segment (start 58.7 15.15741) (end 58.7 13.51759) (width 0.2) (layer "F.Cu") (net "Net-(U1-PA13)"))
 (segment (start 58.7 13.51759) (end 56.63241 11.45) (width 0.2) (layer "F.Cu") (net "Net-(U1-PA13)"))
 (segment (start 57.60741 16.25) (end 58.7 15.15741) (width 0.2) (layer "F.Cu") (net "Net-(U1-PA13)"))
 (segment (start 56.63241 11.45) (end 35.565075 11.45) (width 0.2) (layer "F.Cu") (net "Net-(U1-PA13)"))
 (segment (start 35.565075 11.45) (end 34.95 12.065076) (width 0.2) (layer "F.Cu") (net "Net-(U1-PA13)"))
 (segment (start 34.95 12.934925) (end 39.949389 17.934314) (width 0.2) (layer "F.Cu") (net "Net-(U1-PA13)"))
 (via (at 45.5 17.934314) (size 0.6) (drill 0.3) (layers "F.Cu" "B.Cu") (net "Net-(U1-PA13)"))
 (segment (start 45.834314 22.4) (end 44.834314 21.4) (width 0.2) (layer "B.Cu") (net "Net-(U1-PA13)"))
 (segment (start 49.8 21.461522) (end 49.8 22.538478) (width 0.2) (layer "B.Cu") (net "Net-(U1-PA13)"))
 (segment (start 49.8 22.538478) (end 49.038478 23.3) (width 0.2) (layer "B.Cu") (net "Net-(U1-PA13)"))
 (segment (start 42.6 21.4) (end 41.5 22.5) (width 0.2) (layer "B.Cu") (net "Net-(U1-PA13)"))
 (segment (start 49.038478 20.7) (end 49.8 21.461522) (width 0.2) (layer "B.Cu") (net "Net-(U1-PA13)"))
 (segment (start 45.5 17.934314) (end 45.5 18.5) (width 0.2) (layer "B.Cu") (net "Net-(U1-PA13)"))
 (segment (start 44.834314 21.4) (end 42.6 21.4) (width 0.2) (layer "B.Cu") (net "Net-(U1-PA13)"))
 (segment (start 47.061522 22.4) (end 45.834314 22.4) (width 0.2) (layer "B.Cu") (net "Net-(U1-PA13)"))
 (segment (start 49.038478 23.3) (end 47.961522 23.3) (width 0.2) (layer "B.Cu") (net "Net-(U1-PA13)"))
 (segment (start 45.5 18.5) (end 44.9 19.1) (width 0.2) (layer "B.Cu") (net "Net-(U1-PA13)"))
 (segment (start 44.9 19.1) (end 44.9 19.334315) (width 0.2) (layer "B.Cu") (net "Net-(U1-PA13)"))
 (segment (start 44.9 19.334315) (end 46.265685 20.7) (width 0.2) (layer "B.Cu") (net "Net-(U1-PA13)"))
 (segment (start 47.961522 23.3) (end 47.061522 22.4) (width 0.2) (layer "B.Cu") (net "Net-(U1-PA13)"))
 (segment (start 46.265685 20.7) (end 49.038478 20.7) (width 0.2) (layer "B.Cu") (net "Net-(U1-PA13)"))
 (segment (start 59.6625 15.75) (end 60.43241 15.75) (width 0.2) (layer "F.Cu") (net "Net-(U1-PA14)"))
 (segment (start 60.7 16.01759) (end 60.7 22.048095) (width 0.2) (layer "F.Cu") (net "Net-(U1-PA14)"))
 (segment (start 60.7 22.048095) (end 55.248095 27.5) (width 0.2) (layer "F.Cu") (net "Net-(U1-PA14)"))
 (segment (start 55.248095 27.5) (end 45 27.5) (width 0.2) (layer "F.Cu") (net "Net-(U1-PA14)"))
 (segment (start 60.43241 15.75) (end 60.7 16.01759) (width 0.2) (layer "F.Cu") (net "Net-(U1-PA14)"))
 (via (at 45 27.5) (size 0.6) (drill 0.3) (layers "F.Cu" "B.Cu") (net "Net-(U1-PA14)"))
 (segment (start 45 27.5) (end 44.5 28) (width 0.2) (layer "B.Cu") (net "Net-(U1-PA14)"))
 (segment (start 44.5 28) (end 41.5 28) (width 0.2) (layer "B.Cu") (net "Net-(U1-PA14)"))
 (segment (start 31.33241 23.6) (end 30.275 23.6) (width 0.2) (layer "F.Cu") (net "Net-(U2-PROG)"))
 (segment (start 32 24.5) (end 32 24.26759) (width 0.2) (layer "F.Cu") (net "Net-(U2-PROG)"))
 (segment (start 32 24.26759) (end 31.33241 23.6) (width 0.2) (layer "F.Cu") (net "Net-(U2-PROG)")))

